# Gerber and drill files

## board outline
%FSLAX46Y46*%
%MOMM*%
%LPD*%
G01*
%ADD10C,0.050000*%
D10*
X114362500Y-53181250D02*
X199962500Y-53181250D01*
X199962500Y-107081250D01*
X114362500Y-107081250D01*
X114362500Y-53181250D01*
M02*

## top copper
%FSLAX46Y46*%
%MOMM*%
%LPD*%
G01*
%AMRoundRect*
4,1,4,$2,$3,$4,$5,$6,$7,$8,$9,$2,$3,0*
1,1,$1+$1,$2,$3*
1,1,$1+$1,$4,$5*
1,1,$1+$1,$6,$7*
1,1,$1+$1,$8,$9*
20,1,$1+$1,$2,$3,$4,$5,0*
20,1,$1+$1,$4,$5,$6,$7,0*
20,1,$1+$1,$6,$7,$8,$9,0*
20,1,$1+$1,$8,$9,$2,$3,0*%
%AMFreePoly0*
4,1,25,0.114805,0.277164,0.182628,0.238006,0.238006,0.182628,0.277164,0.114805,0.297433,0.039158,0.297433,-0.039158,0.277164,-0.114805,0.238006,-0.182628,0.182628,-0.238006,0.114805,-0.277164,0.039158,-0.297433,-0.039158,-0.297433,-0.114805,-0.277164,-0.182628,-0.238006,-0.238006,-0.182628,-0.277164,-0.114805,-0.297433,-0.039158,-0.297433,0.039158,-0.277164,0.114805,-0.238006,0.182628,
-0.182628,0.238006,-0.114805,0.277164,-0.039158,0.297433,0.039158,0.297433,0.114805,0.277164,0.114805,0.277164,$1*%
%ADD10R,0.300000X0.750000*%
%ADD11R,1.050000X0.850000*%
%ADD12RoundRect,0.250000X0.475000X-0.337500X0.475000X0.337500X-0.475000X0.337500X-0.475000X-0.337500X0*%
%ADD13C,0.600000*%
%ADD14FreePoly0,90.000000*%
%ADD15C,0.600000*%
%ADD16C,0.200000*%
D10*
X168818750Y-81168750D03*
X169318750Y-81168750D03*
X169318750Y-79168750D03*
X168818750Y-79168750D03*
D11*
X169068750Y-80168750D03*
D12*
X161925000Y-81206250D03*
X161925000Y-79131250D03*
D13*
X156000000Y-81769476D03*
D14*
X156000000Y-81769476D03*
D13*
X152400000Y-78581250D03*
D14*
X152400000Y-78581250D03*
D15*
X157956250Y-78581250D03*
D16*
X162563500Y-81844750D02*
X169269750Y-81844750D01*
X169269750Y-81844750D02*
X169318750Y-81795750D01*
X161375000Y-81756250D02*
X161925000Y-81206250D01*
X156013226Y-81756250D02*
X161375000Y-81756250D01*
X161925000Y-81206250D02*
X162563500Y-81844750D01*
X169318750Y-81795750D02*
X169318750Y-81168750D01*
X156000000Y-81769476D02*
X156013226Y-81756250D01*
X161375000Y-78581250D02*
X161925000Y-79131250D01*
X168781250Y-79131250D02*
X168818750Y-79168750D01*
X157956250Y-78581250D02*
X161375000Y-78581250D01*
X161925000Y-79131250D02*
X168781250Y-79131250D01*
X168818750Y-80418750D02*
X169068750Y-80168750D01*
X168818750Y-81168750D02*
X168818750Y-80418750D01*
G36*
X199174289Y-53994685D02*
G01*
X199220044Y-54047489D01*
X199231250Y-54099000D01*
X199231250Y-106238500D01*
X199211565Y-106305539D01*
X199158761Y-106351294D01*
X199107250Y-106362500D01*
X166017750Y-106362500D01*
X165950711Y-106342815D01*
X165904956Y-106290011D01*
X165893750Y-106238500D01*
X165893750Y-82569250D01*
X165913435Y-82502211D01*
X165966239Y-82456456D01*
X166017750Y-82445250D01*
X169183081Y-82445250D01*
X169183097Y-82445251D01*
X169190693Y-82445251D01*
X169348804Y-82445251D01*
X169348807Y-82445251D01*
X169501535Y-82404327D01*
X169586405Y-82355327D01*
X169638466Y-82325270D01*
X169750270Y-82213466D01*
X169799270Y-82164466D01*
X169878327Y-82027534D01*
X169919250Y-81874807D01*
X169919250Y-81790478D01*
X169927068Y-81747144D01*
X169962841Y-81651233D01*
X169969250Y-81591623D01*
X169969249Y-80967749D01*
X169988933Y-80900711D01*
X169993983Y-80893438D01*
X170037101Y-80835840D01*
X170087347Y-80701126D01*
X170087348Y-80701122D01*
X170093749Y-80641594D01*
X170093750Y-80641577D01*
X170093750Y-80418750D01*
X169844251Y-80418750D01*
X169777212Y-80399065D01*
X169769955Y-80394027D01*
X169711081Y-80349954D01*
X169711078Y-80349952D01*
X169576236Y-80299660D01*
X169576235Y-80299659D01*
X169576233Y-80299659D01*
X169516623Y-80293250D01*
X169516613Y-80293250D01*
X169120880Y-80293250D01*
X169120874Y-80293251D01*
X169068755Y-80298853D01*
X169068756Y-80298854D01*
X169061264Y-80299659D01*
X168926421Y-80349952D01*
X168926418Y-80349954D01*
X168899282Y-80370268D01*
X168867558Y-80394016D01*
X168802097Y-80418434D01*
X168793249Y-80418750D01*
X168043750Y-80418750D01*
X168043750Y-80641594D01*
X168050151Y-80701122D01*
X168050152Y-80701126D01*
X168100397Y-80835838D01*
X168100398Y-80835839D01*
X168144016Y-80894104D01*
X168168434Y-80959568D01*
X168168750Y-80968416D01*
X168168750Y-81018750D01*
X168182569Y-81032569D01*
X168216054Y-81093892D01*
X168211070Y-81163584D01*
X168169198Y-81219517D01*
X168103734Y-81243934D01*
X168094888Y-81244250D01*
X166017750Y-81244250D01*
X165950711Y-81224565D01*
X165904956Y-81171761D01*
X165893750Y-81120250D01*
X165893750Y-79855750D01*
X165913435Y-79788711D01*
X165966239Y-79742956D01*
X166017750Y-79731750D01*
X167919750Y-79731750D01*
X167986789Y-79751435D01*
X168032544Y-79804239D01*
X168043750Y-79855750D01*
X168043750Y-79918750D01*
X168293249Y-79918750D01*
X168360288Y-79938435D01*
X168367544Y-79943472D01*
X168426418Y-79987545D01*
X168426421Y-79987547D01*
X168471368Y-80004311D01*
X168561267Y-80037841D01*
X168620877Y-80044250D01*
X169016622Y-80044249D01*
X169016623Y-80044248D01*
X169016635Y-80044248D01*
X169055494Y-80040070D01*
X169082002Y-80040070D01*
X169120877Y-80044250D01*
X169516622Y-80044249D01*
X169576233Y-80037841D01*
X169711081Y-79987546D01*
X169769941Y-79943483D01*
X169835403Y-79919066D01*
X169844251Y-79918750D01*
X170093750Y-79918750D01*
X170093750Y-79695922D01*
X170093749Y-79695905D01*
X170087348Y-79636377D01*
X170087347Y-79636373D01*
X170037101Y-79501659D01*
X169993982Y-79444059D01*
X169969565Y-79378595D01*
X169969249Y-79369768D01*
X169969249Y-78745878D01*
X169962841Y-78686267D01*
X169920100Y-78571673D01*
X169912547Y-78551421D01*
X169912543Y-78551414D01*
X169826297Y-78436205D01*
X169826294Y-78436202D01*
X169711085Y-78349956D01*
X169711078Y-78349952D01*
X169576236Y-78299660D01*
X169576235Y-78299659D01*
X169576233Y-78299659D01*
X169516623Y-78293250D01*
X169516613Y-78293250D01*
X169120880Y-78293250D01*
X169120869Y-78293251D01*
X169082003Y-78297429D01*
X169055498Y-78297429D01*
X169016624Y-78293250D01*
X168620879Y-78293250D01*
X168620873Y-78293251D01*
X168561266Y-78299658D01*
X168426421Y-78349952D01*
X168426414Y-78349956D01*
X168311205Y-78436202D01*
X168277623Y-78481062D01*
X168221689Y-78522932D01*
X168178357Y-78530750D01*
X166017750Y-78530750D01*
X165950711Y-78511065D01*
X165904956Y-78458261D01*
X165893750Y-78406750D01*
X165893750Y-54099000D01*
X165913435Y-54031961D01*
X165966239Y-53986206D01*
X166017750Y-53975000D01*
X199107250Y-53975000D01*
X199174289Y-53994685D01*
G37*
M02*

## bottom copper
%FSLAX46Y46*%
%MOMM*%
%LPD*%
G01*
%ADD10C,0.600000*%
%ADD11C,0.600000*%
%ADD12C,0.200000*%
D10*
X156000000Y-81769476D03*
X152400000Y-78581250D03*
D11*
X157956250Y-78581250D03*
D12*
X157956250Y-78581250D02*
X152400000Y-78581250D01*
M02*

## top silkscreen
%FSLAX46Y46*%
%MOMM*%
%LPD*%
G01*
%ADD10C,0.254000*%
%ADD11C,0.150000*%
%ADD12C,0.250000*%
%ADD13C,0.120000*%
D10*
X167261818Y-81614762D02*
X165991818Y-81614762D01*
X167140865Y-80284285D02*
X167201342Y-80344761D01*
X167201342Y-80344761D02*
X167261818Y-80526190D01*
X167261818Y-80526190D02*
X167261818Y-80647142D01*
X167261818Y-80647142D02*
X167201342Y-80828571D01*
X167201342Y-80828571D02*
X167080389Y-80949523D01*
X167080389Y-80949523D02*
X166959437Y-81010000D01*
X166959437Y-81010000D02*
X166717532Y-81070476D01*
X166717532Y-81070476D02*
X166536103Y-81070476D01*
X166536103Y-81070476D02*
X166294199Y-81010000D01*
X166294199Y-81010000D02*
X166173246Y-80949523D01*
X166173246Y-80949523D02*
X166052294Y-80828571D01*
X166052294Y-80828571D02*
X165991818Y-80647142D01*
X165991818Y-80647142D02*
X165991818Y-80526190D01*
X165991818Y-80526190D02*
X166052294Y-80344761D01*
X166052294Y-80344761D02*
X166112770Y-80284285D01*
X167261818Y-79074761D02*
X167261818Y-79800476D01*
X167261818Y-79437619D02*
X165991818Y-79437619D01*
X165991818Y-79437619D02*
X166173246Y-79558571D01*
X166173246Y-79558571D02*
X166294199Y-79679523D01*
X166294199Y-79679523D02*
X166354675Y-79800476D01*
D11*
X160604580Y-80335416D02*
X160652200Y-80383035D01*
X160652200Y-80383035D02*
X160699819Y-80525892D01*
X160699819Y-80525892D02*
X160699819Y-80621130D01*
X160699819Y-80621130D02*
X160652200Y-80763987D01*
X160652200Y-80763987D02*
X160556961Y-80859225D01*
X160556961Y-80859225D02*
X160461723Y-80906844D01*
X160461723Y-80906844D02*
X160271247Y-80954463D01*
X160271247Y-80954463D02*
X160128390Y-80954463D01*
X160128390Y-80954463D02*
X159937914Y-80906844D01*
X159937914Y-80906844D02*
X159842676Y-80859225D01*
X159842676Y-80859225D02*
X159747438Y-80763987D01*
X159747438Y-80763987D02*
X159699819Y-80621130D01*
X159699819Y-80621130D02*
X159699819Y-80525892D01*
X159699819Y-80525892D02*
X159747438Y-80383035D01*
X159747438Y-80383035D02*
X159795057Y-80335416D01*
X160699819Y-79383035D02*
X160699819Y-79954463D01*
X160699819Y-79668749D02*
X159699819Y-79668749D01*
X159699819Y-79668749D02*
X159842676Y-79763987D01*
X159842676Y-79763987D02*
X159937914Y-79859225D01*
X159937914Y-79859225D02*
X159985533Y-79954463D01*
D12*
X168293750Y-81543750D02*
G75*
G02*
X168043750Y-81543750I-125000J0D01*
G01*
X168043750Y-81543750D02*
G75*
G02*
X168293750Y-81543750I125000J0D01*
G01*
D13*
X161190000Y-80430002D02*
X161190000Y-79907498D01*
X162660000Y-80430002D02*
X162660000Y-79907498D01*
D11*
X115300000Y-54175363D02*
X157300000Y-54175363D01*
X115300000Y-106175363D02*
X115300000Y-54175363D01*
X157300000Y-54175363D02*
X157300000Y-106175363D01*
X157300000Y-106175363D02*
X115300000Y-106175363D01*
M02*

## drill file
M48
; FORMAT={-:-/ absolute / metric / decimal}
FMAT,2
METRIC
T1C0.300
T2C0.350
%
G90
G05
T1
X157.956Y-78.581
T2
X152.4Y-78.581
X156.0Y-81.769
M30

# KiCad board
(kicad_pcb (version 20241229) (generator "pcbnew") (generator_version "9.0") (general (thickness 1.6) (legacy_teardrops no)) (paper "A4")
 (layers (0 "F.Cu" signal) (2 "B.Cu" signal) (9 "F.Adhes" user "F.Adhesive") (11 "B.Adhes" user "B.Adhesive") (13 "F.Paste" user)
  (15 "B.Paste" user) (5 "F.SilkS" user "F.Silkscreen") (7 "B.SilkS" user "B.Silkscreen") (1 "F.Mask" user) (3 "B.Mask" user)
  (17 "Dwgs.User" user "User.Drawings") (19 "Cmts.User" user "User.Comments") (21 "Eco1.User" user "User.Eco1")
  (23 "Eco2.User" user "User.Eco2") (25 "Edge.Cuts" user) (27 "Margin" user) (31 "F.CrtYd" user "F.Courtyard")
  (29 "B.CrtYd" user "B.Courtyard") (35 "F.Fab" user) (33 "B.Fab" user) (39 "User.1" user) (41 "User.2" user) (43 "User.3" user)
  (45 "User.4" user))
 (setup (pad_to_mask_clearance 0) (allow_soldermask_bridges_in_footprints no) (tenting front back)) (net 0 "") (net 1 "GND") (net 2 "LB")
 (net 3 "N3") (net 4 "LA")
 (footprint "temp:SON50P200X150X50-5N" (layer "F.Cu") (at 169.06875 80.16875 90)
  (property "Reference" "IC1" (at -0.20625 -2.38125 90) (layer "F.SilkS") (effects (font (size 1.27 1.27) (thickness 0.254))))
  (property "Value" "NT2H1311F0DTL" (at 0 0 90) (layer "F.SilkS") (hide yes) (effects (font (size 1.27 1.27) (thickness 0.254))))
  (fp_circle (center -1.375 -0.9) (end -1.375 -0.775) (stroke (width 0.25) (type solid)) (fill no) (layer "F.SilkS"))
  (pad "1" smd rect (at -1 -0.25 180) (size 0.3 0.75) (layers "F.Cu" "F.Mask" "F.Paste") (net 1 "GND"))
  (pad "2" smd rect (at -1 0.25 180) (size 0.3 0.75) (layers "F.Cu" "F.Mask" "F.Paste") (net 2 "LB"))
  (pad "3" smd rect (at 1 0.25 180) (size 0.3 0.75) (layers "F.Cu" "F.Mask" "F.Paste") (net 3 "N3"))
  (pad "4" smd rect (at 1 -0.25 180) (size 0.3 0.75) (layers "F.Cu" "F.Mask" "F.Paste") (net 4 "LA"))
  (pad "5" smd rect (at 0 0 90) (size 0.85 1.05) (layers "F.Cu" "F.Mask" "F.Paste") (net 1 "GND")))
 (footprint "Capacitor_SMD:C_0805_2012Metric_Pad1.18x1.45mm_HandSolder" (layer "F.Cu") (at 161.925 80.16875 90)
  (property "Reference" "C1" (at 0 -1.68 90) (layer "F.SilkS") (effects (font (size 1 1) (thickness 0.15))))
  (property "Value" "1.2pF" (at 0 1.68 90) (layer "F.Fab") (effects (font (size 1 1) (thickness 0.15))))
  (fp_line (start -0.261252 -0.735) (end 0.261252 -0.735) (stroke (width 0.12) (type solid)) (layer "F.SilkS"))
  (fp_line (start -0.261252 0.735) (end 0.261252 0.735) (stroke (width 0.12) (type solid)) (layer "F.SilkS"))
  (pad "1" smd roundrect (at -1.0375 0 90) (size 1.175 1.45) (layers "F.Cu" "F.Mask" "F.Paste") (roundrect_rratio 0.212766) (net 2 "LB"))
  (pad "2" smd roundrect (at 1.0375 0 90) (size 1.175 1.45) (layers "F.Cu" "F.Mask" "F.Paste") (roundrect_rratio 0.212766) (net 4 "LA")))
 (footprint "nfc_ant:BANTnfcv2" (layer "F.Cu") (at 116.3 105.175363 90)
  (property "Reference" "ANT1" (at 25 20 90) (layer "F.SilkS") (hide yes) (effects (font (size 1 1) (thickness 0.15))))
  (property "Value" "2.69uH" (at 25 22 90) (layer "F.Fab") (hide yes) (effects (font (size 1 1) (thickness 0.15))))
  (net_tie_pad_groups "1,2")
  (fp_line (start 51 -1) (end 51 41) (stroke (width 0.15) (type solid)) (layer "F.SilkS"))
  (fp_line (start -1 -1) (end 51 -1) (stroke (width 0.15) (type solid)) (layer "F.SilkS"))
  (fp_line (start 51 41) (end -1 41) (stroke (width 0.15) (type solid)) (layer "F.SilkS"))
  (fp_line (start -1 41) (end -1 -1) (stroke (width 0.15) (type solid)) (layer "F.SilkS"))
  (pad "1" thru_hole circle (at 23.405887 39.7 90) (size 0.6 0.6) (drill 0.35) (layers "*.Cu" "*.Mask") (remove_unused_layers no)
   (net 2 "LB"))
  (pad "1" smd custom (at 23.405887 39.7 90) (size 0.6 0.6) (layers "F.Cu") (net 2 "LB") (zone_connect 0) (thermal_bridge_angle 90)
   (options (clearance outline) (anchor circle)) (primitives))
  (pad "2" thru_hole circle (at 26.594113 36.1 90) (size 0.6 0.6) (drill 0.35) (layers "*.Cu" "*.Mask") (remove_unused_layers no)
   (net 4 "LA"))
  (pad "2" smd custom (at 26.594113 36.1 90) (size 0.6 0.6) (layers "F.Cu") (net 4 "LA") (zone_connect 0) (thermal_bridge_angle 90)
   (options (clearance outline) (anchor circle)) (primitives)))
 (gr_rect (start 114.3625 53.18125) (end 199.9625 107.08125) (stroke (width 0.05) (type solid)) (fill no) (layer "Edge.Cuts"))
 (segment (start 162.5635 81.84475) (end 169.26975 81.84475) (width 0.2) (layer "F.Cu") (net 2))
 (segment (start 169.26975 81.84475) (end 169.31875 81.79575) (width 0.2) (layer "F.Cu") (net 2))
 (segment (start 161.375 81.75625) (end 161.925 81.20625) (width 0.2) (layer "F.Cu") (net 2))
 (segment (start 156.013226 81.75625) (end 161.375 81.75625) (width 0.2) (layer "F.Cu") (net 2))
 (segment (start 161.925 81.20625) (end 162.5635 81.84475) (width 0.2) (layer "F.Cu") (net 2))
 (segment (start 169.31875 81.79575) (end 169.31875 81.16875) (width 0.2) (layer "F.Cu") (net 2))
 (segment (start 156 81.769476) (end 156.013226 81.75625) (width 0.2) (layer "F.Cu") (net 2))
 (segment (start 161.375 78.58125) (end 161.925 79.13125) (width 0.2) (layer "F.Cu") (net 4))
 (segment (start 168.78125 79.13125) (end 168.81875 79.16875) (width 0.2) (layer "F.Cu") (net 4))
 (segment (start 157.95625 78.58125) (end 161.375 78.58125) (width 0.2) (layer "F.Cu") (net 4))
 (segment (start 161.925 79.13125) (end 168.78125 79.13125) (width 0.2) (layer "F.Cu") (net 4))
 (via (at 157.95625 78.58125) (size 0.6) (drill 0.3) (layers "F.Cu" "B.Cu") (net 4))
 (segment (start 157.95625 78.58125) (end 152.4 78.58125) (width 0.2) (layer "B.Cu") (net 4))
 (segment (start 168.81875 80.41875) (end 169.06875 80.16875) (width 0.2) (layer "F.Cu") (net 1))
 (segment (start 168.81875 81.16875) (end 168.81875 80.41875) (width 0.2) (layer "F.Cu") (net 1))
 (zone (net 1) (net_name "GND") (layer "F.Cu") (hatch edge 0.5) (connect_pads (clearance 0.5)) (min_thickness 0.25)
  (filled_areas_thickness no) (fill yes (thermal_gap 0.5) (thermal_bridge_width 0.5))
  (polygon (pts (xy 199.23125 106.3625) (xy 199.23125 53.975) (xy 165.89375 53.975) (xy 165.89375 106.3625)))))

